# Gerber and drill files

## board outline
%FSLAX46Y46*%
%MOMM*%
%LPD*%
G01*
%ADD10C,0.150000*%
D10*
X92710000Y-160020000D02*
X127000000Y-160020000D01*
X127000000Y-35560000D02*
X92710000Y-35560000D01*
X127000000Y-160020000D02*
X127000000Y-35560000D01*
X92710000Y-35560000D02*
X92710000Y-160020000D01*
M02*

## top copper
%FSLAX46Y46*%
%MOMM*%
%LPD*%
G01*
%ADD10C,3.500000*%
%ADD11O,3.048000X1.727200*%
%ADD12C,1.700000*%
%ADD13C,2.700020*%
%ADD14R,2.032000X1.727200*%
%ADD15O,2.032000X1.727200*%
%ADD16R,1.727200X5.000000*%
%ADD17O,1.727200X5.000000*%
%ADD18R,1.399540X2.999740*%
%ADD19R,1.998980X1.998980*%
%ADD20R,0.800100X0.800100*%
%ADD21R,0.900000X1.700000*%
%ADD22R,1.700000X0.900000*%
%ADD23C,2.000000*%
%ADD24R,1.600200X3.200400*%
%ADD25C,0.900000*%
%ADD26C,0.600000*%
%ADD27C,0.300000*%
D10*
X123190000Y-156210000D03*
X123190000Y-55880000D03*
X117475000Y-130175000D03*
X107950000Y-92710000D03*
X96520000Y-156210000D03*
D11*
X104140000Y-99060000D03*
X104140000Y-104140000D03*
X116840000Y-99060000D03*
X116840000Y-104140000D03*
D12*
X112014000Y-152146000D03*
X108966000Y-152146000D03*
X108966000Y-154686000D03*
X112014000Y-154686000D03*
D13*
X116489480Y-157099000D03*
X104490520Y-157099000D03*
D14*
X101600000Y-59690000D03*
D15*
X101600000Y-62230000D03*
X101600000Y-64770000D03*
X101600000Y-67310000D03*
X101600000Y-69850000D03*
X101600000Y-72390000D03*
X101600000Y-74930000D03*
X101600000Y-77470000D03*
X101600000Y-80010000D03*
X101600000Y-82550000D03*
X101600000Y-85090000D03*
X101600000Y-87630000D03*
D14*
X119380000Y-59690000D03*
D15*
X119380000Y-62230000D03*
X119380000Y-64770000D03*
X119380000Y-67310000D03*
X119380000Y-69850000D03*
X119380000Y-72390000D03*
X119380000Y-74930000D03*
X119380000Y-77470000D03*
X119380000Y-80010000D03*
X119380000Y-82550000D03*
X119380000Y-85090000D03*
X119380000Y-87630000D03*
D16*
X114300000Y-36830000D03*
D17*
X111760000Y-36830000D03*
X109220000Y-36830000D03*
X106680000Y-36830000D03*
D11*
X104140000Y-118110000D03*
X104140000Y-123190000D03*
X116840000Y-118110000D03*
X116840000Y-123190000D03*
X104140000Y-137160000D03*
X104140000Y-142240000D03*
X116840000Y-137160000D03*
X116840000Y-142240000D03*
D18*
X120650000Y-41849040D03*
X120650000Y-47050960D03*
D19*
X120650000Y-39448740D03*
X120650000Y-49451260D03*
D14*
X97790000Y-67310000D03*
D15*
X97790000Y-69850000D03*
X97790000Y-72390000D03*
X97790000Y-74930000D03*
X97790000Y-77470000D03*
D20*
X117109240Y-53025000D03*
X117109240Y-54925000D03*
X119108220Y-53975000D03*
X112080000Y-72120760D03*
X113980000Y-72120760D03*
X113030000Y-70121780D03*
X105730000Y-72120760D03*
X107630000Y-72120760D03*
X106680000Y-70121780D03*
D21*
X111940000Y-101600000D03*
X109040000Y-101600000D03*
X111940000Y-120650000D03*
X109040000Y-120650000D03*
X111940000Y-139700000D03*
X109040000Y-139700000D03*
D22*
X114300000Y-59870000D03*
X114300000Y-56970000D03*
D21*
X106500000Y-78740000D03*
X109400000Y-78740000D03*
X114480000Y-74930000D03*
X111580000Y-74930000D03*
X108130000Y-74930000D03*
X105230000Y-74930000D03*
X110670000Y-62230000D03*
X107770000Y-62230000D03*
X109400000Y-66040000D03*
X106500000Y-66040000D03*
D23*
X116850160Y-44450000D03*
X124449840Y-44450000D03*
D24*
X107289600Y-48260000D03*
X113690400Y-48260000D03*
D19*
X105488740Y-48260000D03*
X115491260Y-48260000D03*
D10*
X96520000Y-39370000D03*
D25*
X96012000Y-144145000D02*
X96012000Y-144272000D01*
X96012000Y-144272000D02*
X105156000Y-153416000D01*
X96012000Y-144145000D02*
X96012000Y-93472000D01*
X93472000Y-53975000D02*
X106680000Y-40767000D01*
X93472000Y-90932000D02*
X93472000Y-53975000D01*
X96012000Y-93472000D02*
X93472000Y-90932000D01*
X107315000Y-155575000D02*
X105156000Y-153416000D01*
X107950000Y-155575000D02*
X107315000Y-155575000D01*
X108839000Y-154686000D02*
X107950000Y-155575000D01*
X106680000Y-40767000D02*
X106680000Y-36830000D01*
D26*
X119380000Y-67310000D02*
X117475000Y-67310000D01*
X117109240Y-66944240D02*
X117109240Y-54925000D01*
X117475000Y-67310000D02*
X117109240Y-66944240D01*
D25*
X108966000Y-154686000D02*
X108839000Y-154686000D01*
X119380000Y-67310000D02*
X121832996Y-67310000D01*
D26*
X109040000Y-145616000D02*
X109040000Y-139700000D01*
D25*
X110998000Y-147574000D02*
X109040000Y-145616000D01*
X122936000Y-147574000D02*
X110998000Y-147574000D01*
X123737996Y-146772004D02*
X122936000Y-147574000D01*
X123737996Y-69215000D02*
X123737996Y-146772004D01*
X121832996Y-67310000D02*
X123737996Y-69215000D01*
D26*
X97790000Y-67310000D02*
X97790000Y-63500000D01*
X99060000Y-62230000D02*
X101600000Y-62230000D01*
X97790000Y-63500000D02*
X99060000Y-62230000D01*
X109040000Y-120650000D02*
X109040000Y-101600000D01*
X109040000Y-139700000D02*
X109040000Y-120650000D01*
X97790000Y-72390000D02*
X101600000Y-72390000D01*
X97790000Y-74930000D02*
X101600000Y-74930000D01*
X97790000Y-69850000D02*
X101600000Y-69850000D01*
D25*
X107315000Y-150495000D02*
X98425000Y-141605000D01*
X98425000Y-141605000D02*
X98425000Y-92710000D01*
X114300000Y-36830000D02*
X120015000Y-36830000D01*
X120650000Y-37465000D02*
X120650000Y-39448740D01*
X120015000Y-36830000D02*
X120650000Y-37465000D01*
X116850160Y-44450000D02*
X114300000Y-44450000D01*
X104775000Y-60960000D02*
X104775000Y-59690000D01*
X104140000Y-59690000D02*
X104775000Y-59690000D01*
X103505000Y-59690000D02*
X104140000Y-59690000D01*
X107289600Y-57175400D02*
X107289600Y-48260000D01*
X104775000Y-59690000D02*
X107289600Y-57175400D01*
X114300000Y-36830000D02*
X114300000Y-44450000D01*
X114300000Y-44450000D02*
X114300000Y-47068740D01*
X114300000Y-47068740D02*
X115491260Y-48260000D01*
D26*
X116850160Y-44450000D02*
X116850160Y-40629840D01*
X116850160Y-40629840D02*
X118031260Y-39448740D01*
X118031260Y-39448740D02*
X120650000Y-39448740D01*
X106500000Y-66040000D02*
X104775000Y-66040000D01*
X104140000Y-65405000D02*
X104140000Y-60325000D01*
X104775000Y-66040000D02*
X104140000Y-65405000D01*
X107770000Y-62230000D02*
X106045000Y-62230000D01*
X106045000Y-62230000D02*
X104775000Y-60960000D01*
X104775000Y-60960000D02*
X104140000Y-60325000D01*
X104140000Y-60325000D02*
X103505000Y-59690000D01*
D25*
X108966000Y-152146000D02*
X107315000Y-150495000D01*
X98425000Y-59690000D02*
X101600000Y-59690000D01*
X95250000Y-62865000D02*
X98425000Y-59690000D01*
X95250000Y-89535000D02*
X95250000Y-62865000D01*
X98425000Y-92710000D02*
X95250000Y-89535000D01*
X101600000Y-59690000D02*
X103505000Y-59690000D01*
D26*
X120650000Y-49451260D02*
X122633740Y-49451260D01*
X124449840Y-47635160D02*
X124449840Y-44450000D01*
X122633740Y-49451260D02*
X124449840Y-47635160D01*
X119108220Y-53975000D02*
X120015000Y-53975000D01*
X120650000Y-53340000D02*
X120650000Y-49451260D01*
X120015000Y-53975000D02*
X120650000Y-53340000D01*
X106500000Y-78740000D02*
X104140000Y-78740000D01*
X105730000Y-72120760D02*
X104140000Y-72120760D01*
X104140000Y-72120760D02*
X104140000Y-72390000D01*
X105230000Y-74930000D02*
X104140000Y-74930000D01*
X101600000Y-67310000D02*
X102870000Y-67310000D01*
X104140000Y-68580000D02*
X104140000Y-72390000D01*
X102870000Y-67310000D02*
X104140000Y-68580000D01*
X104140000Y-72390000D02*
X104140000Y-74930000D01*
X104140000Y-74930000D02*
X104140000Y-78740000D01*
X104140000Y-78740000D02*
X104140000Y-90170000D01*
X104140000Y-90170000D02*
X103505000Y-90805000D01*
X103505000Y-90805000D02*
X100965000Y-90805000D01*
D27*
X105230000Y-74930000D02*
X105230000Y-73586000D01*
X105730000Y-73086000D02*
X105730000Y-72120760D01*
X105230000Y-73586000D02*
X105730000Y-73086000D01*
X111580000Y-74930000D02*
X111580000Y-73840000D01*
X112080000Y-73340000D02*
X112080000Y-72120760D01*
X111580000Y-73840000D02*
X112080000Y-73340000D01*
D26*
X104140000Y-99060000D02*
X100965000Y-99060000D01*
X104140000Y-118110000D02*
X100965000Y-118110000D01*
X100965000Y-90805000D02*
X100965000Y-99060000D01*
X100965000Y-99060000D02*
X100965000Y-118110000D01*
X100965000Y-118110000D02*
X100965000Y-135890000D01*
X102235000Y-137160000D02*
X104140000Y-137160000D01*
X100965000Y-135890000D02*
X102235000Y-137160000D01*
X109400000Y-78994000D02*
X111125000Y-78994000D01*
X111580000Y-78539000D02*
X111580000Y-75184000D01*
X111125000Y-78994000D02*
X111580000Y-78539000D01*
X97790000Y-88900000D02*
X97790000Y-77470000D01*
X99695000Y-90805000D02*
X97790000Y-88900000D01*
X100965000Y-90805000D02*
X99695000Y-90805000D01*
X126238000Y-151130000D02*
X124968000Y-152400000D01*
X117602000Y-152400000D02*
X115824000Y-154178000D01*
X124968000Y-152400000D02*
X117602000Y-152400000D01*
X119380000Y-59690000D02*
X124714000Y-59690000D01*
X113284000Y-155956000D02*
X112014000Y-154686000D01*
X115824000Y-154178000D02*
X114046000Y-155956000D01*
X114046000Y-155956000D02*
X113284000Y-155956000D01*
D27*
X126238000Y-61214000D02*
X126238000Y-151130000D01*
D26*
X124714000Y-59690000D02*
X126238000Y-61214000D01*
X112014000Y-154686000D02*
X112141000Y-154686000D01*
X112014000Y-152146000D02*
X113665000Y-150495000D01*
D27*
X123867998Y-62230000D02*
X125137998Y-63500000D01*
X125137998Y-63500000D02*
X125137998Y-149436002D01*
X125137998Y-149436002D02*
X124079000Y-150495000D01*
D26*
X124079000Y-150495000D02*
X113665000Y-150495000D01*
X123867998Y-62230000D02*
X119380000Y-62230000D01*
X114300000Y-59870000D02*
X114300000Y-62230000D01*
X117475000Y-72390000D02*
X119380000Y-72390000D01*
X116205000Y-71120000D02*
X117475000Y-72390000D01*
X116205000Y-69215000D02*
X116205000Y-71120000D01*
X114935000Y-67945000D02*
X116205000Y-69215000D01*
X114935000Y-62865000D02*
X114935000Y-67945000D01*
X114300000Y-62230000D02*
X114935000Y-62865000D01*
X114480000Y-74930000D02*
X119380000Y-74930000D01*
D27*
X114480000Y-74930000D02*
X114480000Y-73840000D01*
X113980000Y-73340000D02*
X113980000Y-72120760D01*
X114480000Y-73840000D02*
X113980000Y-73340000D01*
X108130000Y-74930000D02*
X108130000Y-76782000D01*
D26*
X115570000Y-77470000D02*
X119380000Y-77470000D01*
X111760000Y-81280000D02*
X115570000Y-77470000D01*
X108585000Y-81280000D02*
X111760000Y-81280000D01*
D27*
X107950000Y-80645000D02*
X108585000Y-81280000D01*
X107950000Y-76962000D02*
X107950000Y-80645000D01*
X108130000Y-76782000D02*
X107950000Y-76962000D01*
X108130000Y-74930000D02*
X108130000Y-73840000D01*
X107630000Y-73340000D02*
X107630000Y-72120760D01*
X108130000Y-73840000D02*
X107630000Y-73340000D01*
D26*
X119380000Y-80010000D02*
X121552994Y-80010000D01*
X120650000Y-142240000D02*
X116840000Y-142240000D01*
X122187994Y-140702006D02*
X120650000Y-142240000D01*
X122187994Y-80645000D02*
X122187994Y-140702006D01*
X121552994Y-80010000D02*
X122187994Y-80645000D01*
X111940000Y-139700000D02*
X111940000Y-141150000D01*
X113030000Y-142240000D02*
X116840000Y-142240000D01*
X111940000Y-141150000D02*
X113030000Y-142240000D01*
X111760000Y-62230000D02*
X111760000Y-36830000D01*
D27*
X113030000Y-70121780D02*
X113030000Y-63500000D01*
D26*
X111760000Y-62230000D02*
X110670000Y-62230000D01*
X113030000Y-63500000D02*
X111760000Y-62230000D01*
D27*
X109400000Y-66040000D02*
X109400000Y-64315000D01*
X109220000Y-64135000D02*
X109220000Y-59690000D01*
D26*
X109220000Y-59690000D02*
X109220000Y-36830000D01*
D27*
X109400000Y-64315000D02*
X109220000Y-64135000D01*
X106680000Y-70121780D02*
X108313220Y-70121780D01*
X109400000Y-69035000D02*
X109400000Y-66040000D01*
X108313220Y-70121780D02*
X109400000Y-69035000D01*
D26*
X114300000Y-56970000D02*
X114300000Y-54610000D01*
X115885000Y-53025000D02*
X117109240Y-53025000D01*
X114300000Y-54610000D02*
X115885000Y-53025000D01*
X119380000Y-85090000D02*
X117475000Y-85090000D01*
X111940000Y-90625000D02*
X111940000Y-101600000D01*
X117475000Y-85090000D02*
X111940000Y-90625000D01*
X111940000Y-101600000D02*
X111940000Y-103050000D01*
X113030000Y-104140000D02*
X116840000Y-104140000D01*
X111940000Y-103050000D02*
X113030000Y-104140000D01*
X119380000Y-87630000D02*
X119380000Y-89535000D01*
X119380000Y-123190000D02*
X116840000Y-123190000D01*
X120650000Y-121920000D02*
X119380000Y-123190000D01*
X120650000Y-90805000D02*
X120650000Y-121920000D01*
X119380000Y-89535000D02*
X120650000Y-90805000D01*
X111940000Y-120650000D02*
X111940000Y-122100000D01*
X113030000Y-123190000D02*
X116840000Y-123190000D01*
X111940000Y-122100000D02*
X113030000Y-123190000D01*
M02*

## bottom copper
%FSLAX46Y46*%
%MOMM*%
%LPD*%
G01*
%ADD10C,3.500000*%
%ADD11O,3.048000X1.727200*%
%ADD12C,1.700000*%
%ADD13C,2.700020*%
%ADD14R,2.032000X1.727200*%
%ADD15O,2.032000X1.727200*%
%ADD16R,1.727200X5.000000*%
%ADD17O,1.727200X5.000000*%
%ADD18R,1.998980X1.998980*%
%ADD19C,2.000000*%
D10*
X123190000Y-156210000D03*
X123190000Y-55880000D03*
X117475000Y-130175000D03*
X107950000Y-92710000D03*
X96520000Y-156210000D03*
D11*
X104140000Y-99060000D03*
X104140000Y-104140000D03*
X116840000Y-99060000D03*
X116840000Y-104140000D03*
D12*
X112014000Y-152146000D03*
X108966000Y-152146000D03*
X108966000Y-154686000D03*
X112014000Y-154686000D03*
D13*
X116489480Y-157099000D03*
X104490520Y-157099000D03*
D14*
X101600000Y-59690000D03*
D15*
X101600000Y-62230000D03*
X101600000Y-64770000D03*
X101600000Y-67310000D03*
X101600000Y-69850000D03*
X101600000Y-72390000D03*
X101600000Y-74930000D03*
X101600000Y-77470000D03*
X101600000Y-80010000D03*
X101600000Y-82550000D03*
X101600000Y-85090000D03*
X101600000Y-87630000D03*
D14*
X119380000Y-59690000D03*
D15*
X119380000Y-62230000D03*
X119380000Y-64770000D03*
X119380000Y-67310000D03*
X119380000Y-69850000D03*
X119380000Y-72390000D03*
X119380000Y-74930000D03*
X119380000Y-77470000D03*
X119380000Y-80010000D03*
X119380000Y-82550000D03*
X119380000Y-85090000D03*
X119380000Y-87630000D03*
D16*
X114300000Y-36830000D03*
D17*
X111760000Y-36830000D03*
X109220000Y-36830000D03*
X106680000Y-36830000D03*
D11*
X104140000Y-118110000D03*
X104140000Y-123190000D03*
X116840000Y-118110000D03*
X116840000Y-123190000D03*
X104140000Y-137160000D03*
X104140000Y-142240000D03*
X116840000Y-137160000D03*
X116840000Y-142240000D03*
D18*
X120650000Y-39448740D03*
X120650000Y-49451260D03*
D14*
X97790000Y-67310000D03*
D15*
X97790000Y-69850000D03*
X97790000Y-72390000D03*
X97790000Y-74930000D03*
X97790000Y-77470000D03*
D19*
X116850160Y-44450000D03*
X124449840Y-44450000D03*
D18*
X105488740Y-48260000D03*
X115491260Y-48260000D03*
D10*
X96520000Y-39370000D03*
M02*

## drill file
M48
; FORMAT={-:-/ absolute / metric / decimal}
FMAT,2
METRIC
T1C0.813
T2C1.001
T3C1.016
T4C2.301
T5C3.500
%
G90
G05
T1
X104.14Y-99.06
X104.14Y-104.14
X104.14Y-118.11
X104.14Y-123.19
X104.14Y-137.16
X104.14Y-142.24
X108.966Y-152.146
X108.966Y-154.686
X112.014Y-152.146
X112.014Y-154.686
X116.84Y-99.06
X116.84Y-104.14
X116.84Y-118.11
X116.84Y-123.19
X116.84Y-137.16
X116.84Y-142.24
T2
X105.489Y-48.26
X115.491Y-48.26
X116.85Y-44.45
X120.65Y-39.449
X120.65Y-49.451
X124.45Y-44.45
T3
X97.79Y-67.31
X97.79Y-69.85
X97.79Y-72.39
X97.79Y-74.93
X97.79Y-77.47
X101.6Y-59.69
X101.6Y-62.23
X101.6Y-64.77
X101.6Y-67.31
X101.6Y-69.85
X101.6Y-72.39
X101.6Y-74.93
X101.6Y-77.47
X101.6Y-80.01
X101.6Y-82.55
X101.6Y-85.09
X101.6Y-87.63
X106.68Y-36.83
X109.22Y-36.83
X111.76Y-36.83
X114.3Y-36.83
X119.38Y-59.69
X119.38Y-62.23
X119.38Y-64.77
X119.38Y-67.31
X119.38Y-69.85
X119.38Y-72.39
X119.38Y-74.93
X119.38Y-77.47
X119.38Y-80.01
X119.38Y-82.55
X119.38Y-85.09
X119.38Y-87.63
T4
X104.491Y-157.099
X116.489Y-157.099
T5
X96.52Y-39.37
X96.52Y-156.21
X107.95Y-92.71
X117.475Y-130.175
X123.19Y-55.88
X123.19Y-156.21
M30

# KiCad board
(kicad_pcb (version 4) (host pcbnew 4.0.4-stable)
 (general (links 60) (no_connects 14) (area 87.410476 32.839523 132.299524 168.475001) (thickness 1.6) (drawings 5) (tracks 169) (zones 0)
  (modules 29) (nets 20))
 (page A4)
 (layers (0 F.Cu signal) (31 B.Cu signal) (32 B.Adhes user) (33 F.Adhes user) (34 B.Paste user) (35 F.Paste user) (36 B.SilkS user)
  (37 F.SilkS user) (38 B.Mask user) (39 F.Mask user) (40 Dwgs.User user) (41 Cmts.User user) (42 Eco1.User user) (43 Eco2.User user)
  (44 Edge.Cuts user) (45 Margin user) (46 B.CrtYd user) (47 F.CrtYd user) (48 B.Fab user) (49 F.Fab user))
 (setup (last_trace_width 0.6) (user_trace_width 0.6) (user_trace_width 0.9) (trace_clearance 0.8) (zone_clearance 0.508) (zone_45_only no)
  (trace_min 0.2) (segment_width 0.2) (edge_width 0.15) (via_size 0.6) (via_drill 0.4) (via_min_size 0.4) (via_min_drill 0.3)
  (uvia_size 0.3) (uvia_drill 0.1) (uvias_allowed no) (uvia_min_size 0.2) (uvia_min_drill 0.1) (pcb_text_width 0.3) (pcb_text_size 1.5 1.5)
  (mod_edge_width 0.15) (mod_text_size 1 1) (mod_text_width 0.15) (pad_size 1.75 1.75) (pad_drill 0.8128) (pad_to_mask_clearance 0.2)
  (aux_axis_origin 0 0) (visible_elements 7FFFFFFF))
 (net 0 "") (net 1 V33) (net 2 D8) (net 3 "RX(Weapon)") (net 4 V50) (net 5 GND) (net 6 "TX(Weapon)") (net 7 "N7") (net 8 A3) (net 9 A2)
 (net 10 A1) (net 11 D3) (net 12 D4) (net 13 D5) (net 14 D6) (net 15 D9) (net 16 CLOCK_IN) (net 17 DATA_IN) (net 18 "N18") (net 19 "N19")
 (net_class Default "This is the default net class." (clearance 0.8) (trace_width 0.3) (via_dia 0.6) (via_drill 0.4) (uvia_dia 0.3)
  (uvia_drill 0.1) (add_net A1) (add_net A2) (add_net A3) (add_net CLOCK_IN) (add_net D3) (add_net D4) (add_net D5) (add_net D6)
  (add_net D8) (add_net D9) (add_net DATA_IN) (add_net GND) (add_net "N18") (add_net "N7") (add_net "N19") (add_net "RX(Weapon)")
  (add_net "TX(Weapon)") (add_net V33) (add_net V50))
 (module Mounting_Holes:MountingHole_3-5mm (layer F.Cu) (at 123.19 156.21)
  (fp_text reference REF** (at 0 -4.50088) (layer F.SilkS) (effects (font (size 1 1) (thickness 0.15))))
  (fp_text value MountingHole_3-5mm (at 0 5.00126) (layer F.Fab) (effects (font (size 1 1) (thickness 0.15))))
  (pad 1 thru_hole circle (at 0 0) (size 3.5 3.5) (drill 3.5) (layers)))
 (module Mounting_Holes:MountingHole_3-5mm (layer F.Cu) (at 123.19 55.88)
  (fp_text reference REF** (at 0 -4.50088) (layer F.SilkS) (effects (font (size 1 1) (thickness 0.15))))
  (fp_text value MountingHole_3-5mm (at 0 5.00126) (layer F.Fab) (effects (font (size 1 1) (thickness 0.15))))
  (pad 1 thru_hole circle (at 0 0) (size 3.5 3.5) (drill 3.5) (layers)))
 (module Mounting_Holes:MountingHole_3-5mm (layer F.Cu) (at 117.475 130.175)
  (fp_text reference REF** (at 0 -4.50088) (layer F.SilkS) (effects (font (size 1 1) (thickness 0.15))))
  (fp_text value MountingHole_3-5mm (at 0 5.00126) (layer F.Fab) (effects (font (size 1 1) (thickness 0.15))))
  (pad 1 thru_hole circle (at 0 0) (size 3.5 3.5) (drill 3.5) (layers)))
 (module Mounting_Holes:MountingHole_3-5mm (layer F.Cu) (at 107.95 92.71)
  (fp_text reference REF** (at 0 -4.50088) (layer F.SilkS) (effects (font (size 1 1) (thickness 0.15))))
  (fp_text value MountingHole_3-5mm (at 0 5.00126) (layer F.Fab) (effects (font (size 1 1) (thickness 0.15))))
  (pad 1 thru_hole circle (at 0 0) (size 3.5 3.5) (drill 3.5) (layers)))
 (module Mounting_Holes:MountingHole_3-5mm (layer F.Cu) (at 96.52 156.21)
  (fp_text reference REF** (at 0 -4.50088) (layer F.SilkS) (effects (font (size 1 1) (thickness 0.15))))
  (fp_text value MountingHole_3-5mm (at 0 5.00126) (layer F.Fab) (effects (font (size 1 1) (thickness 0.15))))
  (pad 1 thru_hole circle (at 0 0) (size 3.5 3.5) (drill 3.5) (layers)))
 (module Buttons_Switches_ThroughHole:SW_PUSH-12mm (layer B.Cu) (at 110.49 101.6 180)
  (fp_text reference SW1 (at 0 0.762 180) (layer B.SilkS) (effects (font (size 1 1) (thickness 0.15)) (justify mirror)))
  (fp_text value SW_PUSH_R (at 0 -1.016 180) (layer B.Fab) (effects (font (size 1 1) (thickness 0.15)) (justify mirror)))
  (pad 1 thru_hole oval (at 6.35 2.54 180) (size 3.048 1.7272) (drill 0.8128) (layers *.Cu *.Mask) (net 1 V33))
  (pad 2 thru_hole oval (at 6.35 -2.54 180) (size 3.048 1.7272) (drill 0.8128) (layers *.Cu *.Mask) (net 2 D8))
  (pad 1 thru_hole oval (at -6.35 2.54 180) (size 3.048 1.7272) (drill 0.8128) (layers *.Cu *.Mask) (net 1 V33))
  (pad 2 thru_hole oval (at -6.35 -2.54 180) (size 3.048 1.7272) (drill 0.8128) (layers *.Cu *.Mask) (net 2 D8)))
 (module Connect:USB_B (layer B.Cu) (at 109.22 152.4 270)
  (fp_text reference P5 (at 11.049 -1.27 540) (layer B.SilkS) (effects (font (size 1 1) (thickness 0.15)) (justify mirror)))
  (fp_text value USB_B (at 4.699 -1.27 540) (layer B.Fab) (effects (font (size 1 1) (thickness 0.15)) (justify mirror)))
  (pad 2 thru_hole circle (at -0.254 -2.794) (size 1.7 1.7) (drill 0.8128) (layers *.Cu *.Mask) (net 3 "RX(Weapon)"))
  (pad 1 thru_hole circle (at -0.254 0.254) (size 1.7 1.7) (drill 0.8128) (layers *.Cu *.Mask) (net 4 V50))
  (pad 4 thru_hole circle (at 2.286 0.254) (size 1.7 1.7) (drill 0.8128) (layers *.Cu *.Mask) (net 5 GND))
  (pad 3 thru_hole circle (at 2.286 -2.794) (size 1.7 1.7) (drill 0.8128) (layers *.Cu *.Mask) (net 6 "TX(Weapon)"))
  (pad 5 thru_hole circle (at 4.699 -7.26948) (size 2.70002 2.70002) (drill 2.30124) (layers *.Cu *.Mask) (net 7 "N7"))
  (pad 5 thru_hole circle (at 4.699 4.72948) (size 2.70002 2.70002) (drill 2.30124) (layers *.Cu *.Mask) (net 7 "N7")))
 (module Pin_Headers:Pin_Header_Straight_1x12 (layer B.Cu) (at 101.6 59.69 180)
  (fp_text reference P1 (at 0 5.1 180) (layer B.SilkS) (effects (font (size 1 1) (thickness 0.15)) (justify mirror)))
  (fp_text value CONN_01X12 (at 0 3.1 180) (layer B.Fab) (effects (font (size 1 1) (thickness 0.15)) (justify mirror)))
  (pad 1 thru_hole rect (at 0 0 180) (size 2.032 1.7272) (drill 1.016) (layers *.Cu *.Mask) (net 4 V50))
  (pad 2 thru_hole oval (at 0 -2.54 180) (size 2.032 1.7272) (drill 1.016) (layers *.Cu *.Mask) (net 5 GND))
  (pad 3 thru_hole oval (at 0 -5.08 180) (size 2.032 1.7272) (drill 1.016) (layers *.Cu *.Mask))
  (pad 4 thru_hole oval (at 0 -7.62 180) (size 2.032 1.7272) (drill 1.016) (layers *.Cu *.Mask) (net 1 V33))
  (pad 5 thru_hole oval (at 0 -10.16 180) (size 2.032 1.7272) (drill 1.016) (layers *.Cu *.Mask) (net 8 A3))
  (pad 6 thru_hole oval (at 0 -12.7 180) (size 2.032 1.7272) (drill 1.016) (layers *.Cu *.Mask) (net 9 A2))
  (pad 7 thru_hole oval (at 0 -15.24 180) (size 2.032 1.7272) (drill 1.016) (layers *.Cu *.Mask) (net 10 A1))
  (pad 8 thru_hole oval (at 0 -17.78 180) (size 2.032 1.7272) (drill 1.016) (layers *.Cu *.Mask))
  (pad 9 thru_hole oval (at 0 -20.32 180) (size 2.032 1.7272) (drill 1.016) (layers *.Cu *.Mask))
  (pad 10 thru_hole oval (at 0 -22.86 180) (size 2.032 1.7272) (drill 1.016) (layers *.Cu *.Mask))
  (pad 11 thru_hole oval (at 0 -25.4 180) (size 2.032 1.7272) (drill 1.016) (layers *.Cu *.Mask))
  (pad 12 thru_hole oval (at 0 -27.94 180) (size 2.032 1.7272) (drill 1.016) (layers *.Cu *.Mask)))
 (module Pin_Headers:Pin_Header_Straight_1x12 (layer B.Cu) (at 119.38 59.69 180)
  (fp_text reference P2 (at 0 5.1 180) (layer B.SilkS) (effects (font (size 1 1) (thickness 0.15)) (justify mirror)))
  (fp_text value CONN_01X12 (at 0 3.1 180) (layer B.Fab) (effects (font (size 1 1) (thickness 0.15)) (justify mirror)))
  (pad 1 thru_hole rect (at 0 0 180) (size 2.032 1.7272) (drill 1.016) (layers *.Cu *.Mask) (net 6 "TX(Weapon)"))
  (pad 2 thru_hole oval (at 0 -2.54 180) (size 2.032 1.7272) (drill 1.016) (layers *.Cu *.Mask) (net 3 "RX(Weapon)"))
  (pad 3 thru_hole oval (at 0 -5.08 180) (size 2.032 1.7272) (drill 1.016) (layers *.Cu *.Mask))
  (pad 4 thru_hole oval (at 0 -7.62 180) (size 2.032 1.7272) (drill 1.016) (layers *.Cu *.Mask) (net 5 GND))
  (pad 5 thru_hole oval (at 0 -10.16 180) (size 2.032 1.7272) (drill 1.016) (layers *.Cu *.Mask))
  (pad 6 thru_hole oval (at 0 -12.7 180) (size 2.032 1.7272) (drill 1.016) (layers *.Cu *.Mask) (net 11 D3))
  (pad 7 thru_hole oval (at 0 -15.24 180) (size 2.032 1.7272) (drill 1.016) (layers *.Cu *.Mask) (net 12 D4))
  (pad 8 thru_hole oval (at 0 -17.78 180) (size 2.032 1.7272) (drill 1.016) (layers *.Cu *.Mask) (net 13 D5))
  (pad 9 thru_hole oval (at 0 -20.32 180) (size 2.032 1.7272) (drill 1.016) (layers *.Cu *.Mask) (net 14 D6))
  (pad 10 thru_hole oval (at 0 -22.86 180) (size 2.032 1.7272) (drill 1.016) (layers *.Cu *.Mask))
  (pad 11 thru_hole oval (at 0 -25.4 180) (size 2.032 1.7272) (drill 1.016) (layers *.Cu *.Mask) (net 2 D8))
  (pad 12 thru_hole oval (at 0 -27.94 180) (size 2.032 1.7272) (drill 1.016) (layers *.Cu *.Mask) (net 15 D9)))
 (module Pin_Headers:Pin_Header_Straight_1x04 (layer F.Cu) (at 114.3 36.83 270)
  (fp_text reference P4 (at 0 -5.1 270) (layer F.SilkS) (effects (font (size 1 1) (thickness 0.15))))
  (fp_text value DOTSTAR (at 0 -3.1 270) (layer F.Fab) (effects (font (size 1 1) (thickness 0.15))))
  (pad 1 thru_hole rect (at 0 0 270) (size 5 1.7272) (drill 1.016) (layers *.Cu *.Mask) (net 4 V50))
  (pad 2 thru_hole oval (at 0 2.54 270) (size 5 1.7272) (drill 1.016) (layers *.Cu *.Mask) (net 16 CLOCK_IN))
  (pad 3 thru_hole oval (at 0 5.08 270) (size 5 1.7272) (drill 1.016) (layers *.Cu *.Mask) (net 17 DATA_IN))
  (pad 4 thru_hole oval (at 0 7.62 270) (size 5 1.7272) (drill 1.016) (layers *.Cu *.Mask) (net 5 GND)))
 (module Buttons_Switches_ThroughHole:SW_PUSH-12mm (layer B.Cu) (at 110.49 120.65 180)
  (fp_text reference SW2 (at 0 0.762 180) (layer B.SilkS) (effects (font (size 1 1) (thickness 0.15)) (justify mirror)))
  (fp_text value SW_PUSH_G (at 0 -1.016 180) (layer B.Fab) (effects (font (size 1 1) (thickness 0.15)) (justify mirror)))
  (pad 1 thru_hole oval (at 6.35 2.54 180) (size 3.048 1.7272) (drill 0.8128) (layers *.Cu *.Mask) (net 1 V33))
  (pad 2 thru_hole oval (at 6.35 -2.54 180) (size 3.048 1.7272) (drill 0.8128) (layers *.Cu *.Mask) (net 15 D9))
  (pad 1 thru_hole oval (at -6.35 2.54 180) (size 3.048 1.7272) (drill 0.8128) (layers *.Cu *.Mask) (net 1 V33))
  (pad 2 thru_hole oval (at -6.35 -2.54 180) (size 3.048 1.7272) (drill 0.8128) (layers *.Cu *.Mask) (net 15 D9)))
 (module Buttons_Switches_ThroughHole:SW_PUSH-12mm (layer B.Cu) (at 110.49 139.7 180)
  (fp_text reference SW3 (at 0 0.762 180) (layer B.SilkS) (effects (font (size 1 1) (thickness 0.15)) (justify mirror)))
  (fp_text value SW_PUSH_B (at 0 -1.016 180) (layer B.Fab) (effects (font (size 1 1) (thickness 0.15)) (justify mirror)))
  (pad 1 thru_hole oval (at 6.35 2.54 180) (size 3.048 1.7272) (drill 0.8128) (layers *.Cu *.Mask) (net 1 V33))
  (pad 2 thru_hole oval (at 6.35 -2.54 180) (size 3.048 1.7272) (drill 0.8128) (layers *.Cu *.Mask) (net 14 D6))
  (pad 1 thru_hole oval (at -6.35 2.54 180) (size 3.048 1.7272) (drill 0.8128) (layers *.Cu *.Mask) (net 1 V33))
  (pad 2 thru_hole oval (at -6.35 -2.54 180) (size 3.048 1.7272) (drill 0.8128) (layers *.Cu *.Mask) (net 14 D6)))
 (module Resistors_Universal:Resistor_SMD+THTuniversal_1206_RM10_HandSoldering (layer F.Cu) (at 120.65 44.45 270)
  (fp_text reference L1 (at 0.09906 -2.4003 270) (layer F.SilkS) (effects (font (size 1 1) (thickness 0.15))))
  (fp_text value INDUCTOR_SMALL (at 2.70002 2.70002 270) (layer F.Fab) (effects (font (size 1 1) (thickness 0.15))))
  (pad 1 smd rect (at -2.60096 0 270) (size 2.99974 1.39954) (layers F.Cu F.Paste F.Mask) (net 4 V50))
  (pad 2 smd rect (at 2.60096 0 270) (size 2.99974 1.39954) (layers F.Cu F.Paste F.Mask) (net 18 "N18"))
  (pad 1 thru_hole rect (at -5.00126 0 270) (size 1.99898 1.99898) (drill 1.00076) (layers *.Cu *.Mask F.SilkS) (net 4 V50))
  (pad 2 thru_hole rect (at 5.00126 0 270) (size 1.99898 1.99898) (drill 1.00076) (layers *.Cu *.Mask F.SilkS) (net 18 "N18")))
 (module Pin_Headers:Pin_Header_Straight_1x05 (layer B.Cu) (at 97.79 67.31 180)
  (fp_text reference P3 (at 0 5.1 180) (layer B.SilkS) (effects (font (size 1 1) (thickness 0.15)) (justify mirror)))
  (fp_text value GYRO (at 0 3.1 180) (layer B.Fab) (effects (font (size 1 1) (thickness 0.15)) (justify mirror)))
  (pad 1 thru_hole rect (at 0 0 180) (size 2.032 1.7272) (drill 1.016) (layers *.Cu *.Mask B.SilkS) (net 5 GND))
  (pad 2 thru_hole oval (at 0 -2.54 180) (size 2.032 1.7272) (drill 1.016) (layers *.Cu *.Mask B.SilkS) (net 8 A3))
  (pad 3 thru_hole oval (at 0 -5.08 180) (size 2.032 1.7272) (drill 1.016) (layers *.Cu *.Mask B.SilkS) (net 9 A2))
  (pad 4 thru_hole oval (at 0 -7.62 180) (size 2.032 1.7272) (drill 1.016) (layers *.Cu *.Mask B.SilkS) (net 10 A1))
  (pad 5 thru_hole oval (at 0 -10.16 180) (size 2.032 1.7272) (drill 1.016) (layers *.Cu *.Mask B.SilkS) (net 1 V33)))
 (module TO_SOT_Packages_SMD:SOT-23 (layer F.Cu) (at 118.11 53.975 270)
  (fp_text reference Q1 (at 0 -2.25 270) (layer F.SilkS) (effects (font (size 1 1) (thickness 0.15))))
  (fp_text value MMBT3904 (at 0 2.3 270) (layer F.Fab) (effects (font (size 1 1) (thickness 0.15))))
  (pad 1 smd rect (at -0.95 1.00076 270) (size 0.8001 0.8001) (layers F.Cu F.Paste F.Mask) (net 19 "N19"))
  (pad 2 smd rect (at 0.95 1.00076 270) (size 0.8001 0.8001) (layers F.Cu F.Paste F.Mask) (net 5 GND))
  (pad 3 smd rect (at 0 -0.99822 270) (size 0.8001 0.8001) (layers F.Cu F.Paste F.Mask) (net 18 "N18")))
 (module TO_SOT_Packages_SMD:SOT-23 (layer F.Cu) (at 113.03 71.12)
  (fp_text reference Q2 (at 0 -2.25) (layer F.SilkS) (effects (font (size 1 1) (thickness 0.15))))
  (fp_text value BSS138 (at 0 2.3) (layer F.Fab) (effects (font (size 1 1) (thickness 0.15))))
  (pad 1 smd rect (at -0.95 1.00076) (size 0.8001 0.8001) (layers F.Cu F.Paste F.Mask) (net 1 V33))
  (pad 2 smd rect (at 0.95 1.00076) (size 0.8001 0.8001) (layers F.Cu F.Paste F.Mask) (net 12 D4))
  (pad 3 smd rect (at 0 -0.99822) (size 0.8001 0.8001) (layers F.Cu F.Paste F.Mask) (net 16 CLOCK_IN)))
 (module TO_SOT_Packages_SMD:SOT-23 (layer F.Cu) (at 106.68 71.12)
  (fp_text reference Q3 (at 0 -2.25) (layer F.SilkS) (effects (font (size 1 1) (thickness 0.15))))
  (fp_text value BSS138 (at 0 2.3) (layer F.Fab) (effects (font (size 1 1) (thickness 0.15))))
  (pad 1 smd rect (at -0.95 1.00076) (size 0.8001 0.8001) (layers F.Cu F.Paste F.Mask) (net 1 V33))
  (pad 2 smd rect (at 0.95 1.00076) (size 0.8001 0.8001) (layers F.Cu F.Paste F.Mask) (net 13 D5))
  (pad 3 smd rect (at 0 -0.99822) (size 0.8001 0.8001) (layers F.Cu F.Paste F.Mask) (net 17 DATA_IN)))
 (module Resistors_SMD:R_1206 (layer F.Cu) (at 110.49 101.6 180)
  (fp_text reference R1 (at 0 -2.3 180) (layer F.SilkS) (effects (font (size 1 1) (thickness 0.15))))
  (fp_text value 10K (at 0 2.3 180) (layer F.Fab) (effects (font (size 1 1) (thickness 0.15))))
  (pad 1 smd rect (at -1.45 0 180) (size 0.9 1.7) (layers F.Cu F.Paste F.Mask) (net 2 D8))
  (pad 2 smd rect (at 1.45 0 180) (size 0.9 1.7) (layers F.Cu F.Paste F.Mask) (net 5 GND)))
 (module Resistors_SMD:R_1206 (layer F.Cu) (at 110.49 120.65 180)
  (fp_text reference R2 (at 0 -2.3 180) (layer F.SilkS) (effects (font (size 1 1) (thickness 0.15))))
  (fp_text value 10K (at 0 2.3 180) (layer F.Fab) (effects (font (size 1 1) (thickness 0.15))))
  (pad 1 smd rect (at -1.45 0 180) (size 0.9 1.7) (layers F.Cu F.Paste F.Mask) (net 15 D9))
  (pad 2 smd rect (at 1.45 0 180) (size 0.9 1.7) (layers F.Cu F.Paste F.Mask) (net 5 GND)))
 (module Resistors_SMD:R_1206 (layer F.Cu) (at 110.49 139.7 180)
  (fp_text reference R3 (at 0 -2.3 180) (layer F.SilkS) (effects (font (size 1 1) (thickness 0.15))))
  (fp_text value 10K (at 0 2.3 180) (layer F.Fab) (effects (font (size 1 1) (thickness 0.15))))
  (pad 1 smd rect (at -1.45 0 180) (size 0.9 1.7) (layers F.Cu F.Paste F.Mask) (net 14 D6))
  (pad 2 smd rect (at 1.45 0 180) (size 0.9 1.7) (layers F.Cu F.Paste F.Mask) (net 5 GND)))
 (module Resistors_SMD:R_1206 (layer F.Cu) (at 114.3 58.42 90)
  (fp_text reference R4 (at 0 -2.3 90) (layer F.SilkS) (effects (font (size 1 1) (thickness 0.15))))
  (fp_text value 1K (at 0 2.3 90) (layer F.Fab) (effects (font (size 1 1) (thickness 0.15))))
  (pad 1 smd rect (at -1.45 0 90) (size 0.9 1.7) (layers F.Cu F.Paste F.Mask) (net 11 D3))
  (pad 2 smd rect (at 1.45 0 90) (size 0.9 1.7) (layers F.Cu F.Paste F.Mask) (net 19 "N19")))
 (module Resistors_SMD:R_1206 (layer F.Cu) (at 107.95 78.74)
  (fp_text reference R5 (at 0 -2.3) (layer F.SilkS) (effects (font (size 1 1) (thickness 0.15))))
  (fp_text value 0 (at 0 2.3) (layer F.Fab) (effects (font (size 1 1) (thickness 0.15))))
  (pad 1 smd rect (at -1.45 0) (size 0.9 1.7) (layers F.Cu F.Paste F.Mask) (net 1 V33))
  (pad 2 smd rect (at 1.45 0) (size 0.9 1.7) (layers F.Cu F.Paste F.Mask) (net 1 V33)))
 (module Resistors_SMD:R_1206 (layer F.Cu) (at 113.03 74.93 180)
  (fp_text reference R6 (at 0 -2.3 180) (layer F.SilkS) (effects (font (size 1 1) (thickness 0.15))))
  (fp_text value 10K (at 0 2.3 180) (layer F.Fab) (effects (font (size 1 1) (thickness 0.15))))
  (pad 1 smd rect (at -1.45 0 180) (size 0.9 1.7) (layers F.Cu F.Paste F.Mask) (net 12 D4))
  (pad 2 smd rect (at 1.45 0 180) (size 0.9 1.7) (layers F.Cu F.Paste F.Mask) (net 1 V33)))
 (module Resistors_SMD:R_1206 (layer F.Cu) (at 106.68 74.93 180)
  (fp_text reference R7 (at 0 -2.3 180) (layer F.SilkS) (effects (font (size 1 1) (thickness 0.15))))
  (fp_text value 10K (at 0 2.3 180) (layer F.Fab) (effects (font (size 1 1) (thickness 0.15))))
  (pad 1 smd rect (at -1.45 0 180) (size 0.9 1.7) (layers F.Cu F.Paste F.Mask) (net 13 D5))
  (pad 2 smd rect (at 1.45 0 180) (size 0.9 1.7) (layers F.Cu F.Paste F.Mask) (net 1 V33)))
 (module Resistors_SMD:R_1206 (layer F.Cu) (at 109.22 62.23 180)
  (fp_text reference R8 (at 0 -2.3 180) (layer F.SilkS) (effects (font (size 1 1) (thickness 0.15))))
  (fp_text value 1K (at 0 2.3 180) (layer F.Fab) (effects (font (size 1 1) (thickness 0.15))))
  (pad 1 smd rect (at -1.45 0 180) (size 0.9 1.7) (layers F.Cu F.Paste F.Mask) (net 16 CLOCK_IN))
  (pad 2 smd rect (at 1.45 0 180) (size 0.9 1.7) (layers F.Cu F.Paste F.Mask) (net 4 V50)))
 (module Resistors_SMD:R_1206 (layer F.Cu) (at 107.95 66.04 180)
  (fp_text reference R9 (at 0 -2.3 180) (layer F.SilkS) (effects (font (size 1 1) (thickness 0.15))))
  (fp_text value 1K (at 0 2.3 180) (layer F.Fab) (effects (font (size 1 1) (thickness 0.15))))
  (pad 1 smd rect (at -1.45 0 180) (size 0.9 1.7) (layers F.Cu F.Paste F.Mask) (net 17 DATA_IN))
  (pad 2 smd rect (at 1.45 0 180) (size 0.9 1.7) (layers F.Cu F.Paste F.Mask) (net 4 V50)))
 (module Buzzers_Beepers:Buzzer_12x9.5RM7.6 (layer B.Cu) (at 120.65 44.45)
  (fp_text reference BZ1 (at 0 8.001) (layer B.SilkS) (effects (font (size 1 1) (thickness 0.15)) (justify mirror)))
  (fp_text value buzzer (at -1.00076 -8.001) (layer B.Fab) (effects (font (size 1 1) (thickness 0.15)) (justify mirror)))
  (pad 1 thru_hole circle (at -3.79984 0) (size 2 2) (drill 1.00076) (layers *.Cu *.Mask B.SilkS) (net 4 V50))
  (pad 2 thru_hole circle (at 3.79984 0) (size 2 2) (drill 1.00076) (layers *.Cu *.Mask B.SilkS) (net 18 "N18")))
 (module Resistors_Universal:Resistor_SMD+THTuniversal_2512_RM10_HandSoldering (layer F.Cu) (at 110.49 48.26)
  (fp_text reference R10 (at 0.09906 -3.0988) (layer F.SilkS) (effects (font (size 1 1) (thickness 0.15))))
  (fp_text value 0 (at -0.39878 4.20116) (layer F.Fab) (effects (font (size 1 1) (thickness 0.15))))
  (pad 1 smd rect (at -3.2004 0) (size 1.6002 3.2004) (layers F.Cu F.Paste F.Mask) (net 4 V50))
  (pad 2 smd rect (at 3.2004 0) (size 1.6002 3.2004) (layers F.Cu F.Paste F.Mask) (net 4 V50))
  (pad 1 thru_hole rect (at -5.00126 0 180) (size 1.99898 1.99898) (drill 1.00076) (layers *.Cu *.Mask F.SilkS) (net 4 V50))
  (pad 2 thru_hole rect (at 5.00126 0 180) (size 1.99898 1.99898) (drill 1.00076) (layers *.Cu *.Mask F.SilkS) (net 4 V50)))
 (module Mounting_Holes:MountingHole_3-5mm (layer F.Cu) (at 96.52 39.37)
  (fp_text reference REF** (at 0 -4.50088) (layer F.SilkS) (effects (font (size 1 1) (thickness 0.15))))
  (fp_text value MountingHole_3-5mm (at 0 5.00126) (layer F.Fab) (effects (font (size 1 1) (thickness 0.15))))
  (pad 1 thru_hole circle (at 0 0) (size 3.5 3.5) (drill 3.5) (layers)))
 (gr_line (start 92.71 160.02) (end 127 160.02) (angle 90) (layer Edge.Cuts) (width 0.15))
 (gr_line (start 127 35.56) (end 92.71 35.56) (angle 90) (layer Edge.Cuts) (width 0.15))
 (gr_line (start 127 160.02) (end 127 35.56) (angle 90) (layer Edge.Cuts) (width 0.15))
 (gr_line (start 92.71 35.56) (end 92.71 160.02) (angle 90) (layer Edge.Cuts) (width 0.15))
 (segment (start 96.012 144.145) (end 96.012 144.272) (width 0.9) (layer F.Cu) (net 5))
 (segment (start 96.012 144.272) (end 105.156 153.416) (width 0.9) (layer F.Cu) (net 5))
 (segment (start 96.012 144.145) (end 96.012 93.472) (width 0.9) (layer F.Cu) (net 5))
 (segment (start 93.472 53.975) (end 106.68 40.767) (width 0.9) (layer F.Cu) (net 5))
 (segment (start 93.472 90.932) (end 93.472 53.975) (width 0.9) (layer F.Cu) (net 5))
 (segment (start 96.012 93.472) (end 93.472 90.932) (width 0.9) (layer F.Cu) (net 5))
 (segment (start 107.315 155.575) (end 105.156 153.416) (width 0.9) (layer F.Cu) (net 5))
 (segment (start 107.95 155.575) (end 107.315 155.575) (width 0.9) (layer F.Cu) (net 5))
 (segment (start 108.839 154.686) (end 107.95 155.575) (width 0.9) (layer F.Cu) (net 5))
 (segment (start 106.68 40.767) (end 106.68 36.83) (width 0.9) (layer F.Cu) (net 5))
 (segment (start 119.38 67.31) (end 117.475 67.31) (width 0.6) (layer F.Cu) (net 5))
 (segment (start 117.10924 66.94424) (end 117.10924 54.925) (width 0.6) (layer F.Cu) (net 5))
 (segment (start 117.475 67.31) (end 117.10924 66.94424) (width 0.6) (layer F.Cu) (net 5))
 (segment (start 108.966 154.686) (end 108.839 154.686) (width 0.9) (layer F.Cu) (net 5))
 (segment (start 119.38 67.31) (end 121.832996 67.31) (width 0.9) (layer F.Cu) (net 5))
 (segment (start 109.04 145.616) (end 109.04 139.7) (width 0.6) (layer F.Cu) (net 5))
 (segment (start 110.998 147.574) (end 109.04 145.616) (width 0.9) (layer F.Cu) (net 5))
 (segment (start 122.936 147.574) (end 110.998 147.574) (width 0.9) (layer F.Cu) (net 5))
 (segment (start 123.737996 146.772004) (end 122.936 147.574) (width 0.9) (layer F.Cu) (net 5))
 (segment (start 123.737996 69.215) (end 123.737996 146.772004) (width 0.9) (layer F.Cu) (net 5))
 (segment (start 121.832996 67.31) (end 123.737996 69.215) (width 0.9) (layer F.Cu) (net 5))
 (segment (start 97.79 67.31) (end 97.79 63.5) (width 0.6) (layer F.Cu) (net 5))
 (segment (start 99.06 62.23) (end 101.6 62.23) (width 0.6) (layer F.Cu) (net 5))
 (segment (start 97.79 63.5) (end 99.06 62.23) (width 0.6) (layer F.Cu) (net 5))
 (segment (start 109.04 120.65) (end 109.04 101.6) (width 0.6) (layer F.Cu) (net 5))
 (segment (start 109.04 139.7) (end 109.04 120.65) (width 0.6) (layer F.Cu) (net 5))
 (segment (start 97.79 72.39) (end 101.6 72.39) (width 0.6) (layer F.Cu) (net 9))
 (segment (start 97.79 74.93) (end 101.6 74.93) (width 0.6) (layer F.Cu) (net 10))
 (segment (start 97.79 69.85) (end 101.6 69.85) (width 0.6) (layer F.Cu) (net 8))
 (segment (start 107.315 150.495) (end 98.425 141.605) (width 0.9) (layer F.Cu) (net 4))
 (segment (start 98.425 141.605) (end 98.425 92.71) (width 0.9) (layer F.Cu) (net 4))
 (segment (start 114.3 36.83) (end 120.015 36.83) (width 0.9) (layer F.Cu) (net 4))
 (segment (start 120.65 37.465) (end 120.65 39.44874) (width 0.9) (layer F.Cu) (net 4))
 (segment (start 120.015 36.83) (end 120.65 37.465) (width 0.9) (layer F.Cu) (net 4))
 (segment (start 116.85016 44.45) (end 114.3 44.45) (width 0.9) (layer F.Cu) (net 4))
 (segment (start 104.775 60.96) (end 104.775 59.69) (width 0.9) (layer F.Cu) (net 4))
 (segment (start 104.14 59.69) (end 104.775 59.69) (width 0.9) (layer F.Cu) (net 4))
 (segment (start 103.505 59.69) (end 104.14 59.69) (width 0.9) (layer F.Cu) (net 4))
 (segment (start 107.2896 57.1754) (end 107.2896 48.26) (width 0.9) (layer F.Cu) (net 4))
 (segment (start 104.775 59.69) (end 107.2896 57.1754) (width 0.9) (layer F.Cu) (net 4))
 (segment (start 114.3 36.83) (end 114.3 44.45) (width 0.9) (layer F.Cu) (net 4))
 (segment (start 114.3 44.45) (end 114.3 47.06874) (width 0.9) (layer F.Cu) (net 4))
 (segment (start 114.3 47.06874) (end 115.49126 48.26) (width 0.9) (layer F.Cu) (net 4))
 (segment (start 116.85016 44.45) (end 116.85016 40.62984) (width 0.6) (layer F.Cu) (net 4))
 (segment (start 116.85016 40.62984) (end 118.03126 39.44874) (width 0.6) (layer F.Cu) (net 4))
 (segment (start 118.03126 39.44874) (end 120.65 39.44874) (width 0.6) (layer F.Cu) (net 4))
 (segment (start 106.5 66.04) (end 104.775 66.04) (width 0.6) (layer F.Cu) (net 4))
 (segment (start 104.14 65.405) (end 104.14 60.325) (width 0.6) (layer F.Cu) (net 4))
 (segment (start 104.775 66.04) (end 104.14 65.405) (width 0.6) (layer F.Cu) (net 4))
 (segment (start 107.77 62.23) (end 106.045 62.23) (width 0.6) (layer F.Cu) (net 4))
 (segment (start 106.045 62.23) (end 104.775 60.96) (width 0.6) (layer F.Cu) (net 4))
 (segment (start 104.775 60.96) (end 104.14 60.325) (width 0.6) (layer F.Cu) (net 4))
 (segment (start 104.14 60.325) (end 103.505 59.69) (width 0.6) (layer F.Cu) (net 4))
 (segment (start 108.966 152.146) (end 107.315 150.495) (width 0.9) (layer F.Cu) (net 4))
 (segment (start 98.425 59.69) (end 101.6 59.69) (width 0.9) (layer F.Cu) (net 4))
 (segment (start 95.25 62.865) (end 98.425 59.69) (width 0.9) (layer F.Cu) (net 4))
 (segment (start 95.25 89.535) (end 95.25 62.865) (width 0.9) (layer F.Cu) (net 4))
 (segment (start 98.425 92.71) (end 95.25 89.535) (width 0.9) (layer F.Cu) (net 4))
 (segment (start 101.6 59.69) (end 103.505 59.69) (width 0.9) (layer F.Cu) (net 4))
 (segment (start 120.65 49.45126) (end 122.63374 49.45126) (width 0.6) (layer F.Cu) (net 18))
 (segment (start 124.44984 47.63516) (end 124.44984 44.45) (width 0.6) (layer F.Cu) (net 18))
 (segment (start 122.63374 49.45126) (end 124.44984 47.63516) (width 0.6) (layer F.Cu) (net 18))
 (segment (start 119.10822 53.975) (end 120.015 53.975) (width 0.6) (layer F.Cu) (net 18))
 (segment (start 120.65 53.34) (end 120.65 49.45126) (width 0.6) (layer F.Cu) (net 18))
 (segment (start 120.015 53.975) (end 120.65 53.34) (width 0.6) (layer F.Cu) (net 18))
 (segment (start 106.5 78.74) (end 104.14 78.74) (width 0.6) (layer F.Cu) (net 1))
 (segment (start 105.73 72.12076) (end 104.14 72.12076) (width 0.6) (layer F.Cu) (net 1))
 (segment (start 104.14 72.12076) (end 104.14 72.39) (width 0.6) (layer F.Cu) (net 1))
 (segment (start 105.23 74.93) (end 104.14 74.93) (width 0.6) (layer F.Cu) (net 1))
 (segment (start 101.6 67.31) (end 102.87 67.31) (width 0.6) (layer F.Cu) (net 1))
 (segment (start 104.14 68.58) (end 104.14 72.39) (width 0.6) (layer F.Cu) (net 1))
 (segment (start 102.87 67.31) (end 104.14 68.58) (width 0.6) (layer F.Cu) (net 1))
 (segment (start 104.14 72.39) (end 104.14 74.93) (width 0.6) (layer F.Cu) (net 1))
 (segment (start 104.14 74.93) (end 104.14 78.74) (width 0.6) (layer F.Cu) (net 1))
 (segment (start 104.14 78.74) (end 104.14 90.17) (width 0.6) (layer F.Cu) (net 1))
 (segment (start 104.14 90.17) (end 103.505 90.805) (width 0.6) (layer F.Cu) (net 1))
 (segment (start 103.505 90.805) (end 100.965 90.805) (width 0.6) (layer F.Cu) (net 1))
 (segment (start 105.23 74.93) (end 105.23 73.586) (width 0.3) (layer F.Cu) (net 1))
 (segment (start 105.73 73.086) (end 105.73 72.12076) (width 0.3) (layer F.Cu) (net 1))
 (segment (start 105.23 73.586) (end 105.73 73.086) (width 0.3) (layer F.Cu) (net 1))
 (segment (start 111.58 74.93) (end 111.58 73.84) (width 0.3) (layer F.Cu) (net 1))
 (segment (start 112.08 73.34) (end 112.08 72.12076) (width 0.3) (layer F.Cu) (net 1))
 (segment (start 111.58 73.84) (end 112.08 73.34) (width 0.3) (layer F.Cu) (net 1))
 (segment (start 104.14 99.06) (end 100.965 99.06) (width 0.6) (layer F.Cu) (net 1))
 (segment (start 104.14 118.11) (end 100.965 118.11) (width 0.6) (layer F.Cu) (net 1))
 (segment (start 100.965 90.805) (end 100.965 99.06) (width 0.6) (layer F.Cu) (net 1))
 (segment (start 100.965 99.06) (end 100.965 118.11) (width 0.6) (layer F.Cu) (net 1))
 (segment (start 100.965 118.11) (end 100.965 135.89) (width 0.6) (layer F.Cu) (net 1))
 (segment (start 102.235 137.16) (end 104.14 137.16) (width 0.6) (layer F.Cu) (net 1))
 (segment (start 100.965 135.89) (end 102.235 137.16) (width 0.6) (layer F.Cu) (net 1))
 (segment (start 109.4 78.994) (end 111.125 78.994) (width 0.6) (layer F.Cu) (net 1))
 (segment (start 111.58 78.539) (end 111.58 75.184) (width 0.6) (layer F.Cu) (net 1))
 (segment (start 111.125 78.994) (end 111.58 78.539) (width 0.6) (layer F.Cu) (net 1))
 (segment (start 97.79 88.9) (end 97.79 77.47) (width 0.6) (layer F.Cu) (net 1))
 (segment (start 99.695 90.805) (end 97.79 88.9) (width 0.6) (layer F.Cu) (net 1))
 (segment (start 100.965 90.805) (end 99.695 90.805) (width 0.6) (layer F.Cu) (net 1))
 (segment (start 126.238 151.13) (end 124.968 152.4) (width 0.6) (layer F.Cu) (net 6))
 (segment (start 117.602 152.4) (end 115.824 154.178) (width 0.6) (layer F.Cu) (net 6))
 (segment (start 124.968 152.4) (end 117.602 152.4) (width 0.6) (layer F.Cu) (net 6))
 (segment (start 119.38 59.69) (end 124.714 59.69) (width 0.6) (layer F.Cu) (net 6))
 (segment (start 113.284 155.956) (end 112.014 154.686) (width 0.6) (layer F.Cu) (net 6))
 (segment (start 115.824 154.178) (end 114.046 155.956) (width 0.6) (layer F.Cu) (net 6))
 (segment (start 114.046 155.956) (end 113.284 155.956) (width 0.6) (layer F.Cu) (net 6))
 (segment (start 126.238 61.214) (end 126.238 151.13) (width 0.3) (layer F.Cu) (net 6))
 (segment (start 124.714 59.69) (end 126.238 61.214) (width 0.6) (layer F.Cu) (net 6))
 (segment (start 112.014 154.686) (end 112.141 154.686) (width 0.6) (layer F.Cu) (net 6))
 (segment (start 112.014 152.146) (end 113.665 150.495) (width 0.6) (layer F.Cu) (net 3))
 (segment (start 123.867998 62.23) (end 125.137998 63.5) (width 0.3) (layer F.Cu) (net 3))
 (segment (start 125.137998 63.5) (end 125.137998 149.436002) (width 0.3) (layer F.Cu) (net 3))
 (segment (start 125.137998 149.436002) (end 124.079 150.495) (width 0.3) (layer F.Cu) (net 3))
 (segment (start 124.079 150.495) (end 113.665 150.495) (width 0.6) (layer F.Cu) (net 3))
 (segment (start 123.867998 62.23) (end 119.38 62.23) (width 0.6) (layer F.Cu) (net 3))
 (segment (start 114.3 59.87) (end 114.3 62.23) (width 0.6) (layer F.Cu) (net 11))
 (segment (start 117.475 72.39) (end 119.38 72.39) (width 0.6) (layer F.Cu) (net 11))
 (segment (start 116.205 71.12) (end 117.475 72.39) (width 0.6) (layer F.Cu) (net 11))
 (segment (start 116.205 69.215) (end 116.205 71.12) (width 0.6) (layer F.Cu) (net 11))
 (segment (start 114.935 67.945) (end 116.205 69.215) (width 0.6) (layer F.Cu) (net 11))
 (segment (start 114.935 62.865) (end 114.935 67.945) (width 0.6) (layer F.Cu) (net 11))
 (segment (start 114.3 62.23) (end 114.935 62.865) (width 0.6) (layer F.Cu) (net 11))
 (segment (start 114.48 74.93) (end 119.38 74.93) (width 0.6) (layer F.Cu) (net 12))
 (segment (start 114.48 74.93) (end 114.48 73.84) (width 0.3) (layer F.Cu) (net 12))
 (segment (start 113.98 73.34) (end 113.98 72.12076) (width 0.3) (layer F.Cu) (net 12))
 (segment (start 114.48 73.84) (end 113.98 73.34) (width 0.3) (layer F.Cu) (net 12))
 (segment (start 108.13 74.93) (end 108.13 76.782) (width 0.3) (layer F.Cu) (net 13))
 (segment (start 115.57 77.47) (end 119.38 77.47) (width 0.6) (layer F.Cu) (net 13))
 (segment (start 111.76 81.28) (end 115.57 77.47) (width 0.6) (layer F.Cu) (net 13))
 (segment (start 108.585 81.28) (end 111.76 81.28) (width 0.6) (layer F.Cu) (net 13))
 (segment (start 107.95 80.645) (end 108.585 81.28) (width 0.3) (layer F.Cu) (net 13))
 (segment (start 107.95 76.962) (end 107.95 80.645) (width 0.3) (layer F.Cu) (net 13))
 (segment (start 108.13 76.782) (end 107.95 76.962) (width 0.3) (layer F.Cu) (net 13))
 (segment (start 108.13 74.93) (end 108.13 73.84) (width 0.3) (layer F.Cu) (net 13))
 (segment (start 107.63 73.34) (end 107.63 72.12076) (width 0.3) (layer F.Cu) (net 13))
 (segment (start 108.13 73.84) (end 107.63 73.34) (width 0.3) (layer F.Cu) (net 13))
 (segment (start 119.38 80.01) (end 121.552994 80.01) (width 0.6) (layer F.Cu) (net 14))
 (segment (start 120.65 142.24) (end 116.84 142.24) (width 0.6) (layer F.Cu) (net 14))
 (segment (start 122.187994 140.702006) (end 120.65 142.24) (width 0.6) (layer F.Cu) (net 14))
 (segment (start 122.187994 80.645) (end 122.187994 140.702006) (width 0.6) (layer F.Cu) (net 14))
 (segment (start 121.552994 80.01) (end 122.187994 80.645) (width 0.6) (layer F.Cu) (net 14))
 (segment (start 111.94 139.7) (end 111.94 141.15) (width 0.6) (layer F.Cu) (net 14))
 (segment (start 113.03 142.24) (end 116.84 142.24) (width 0.6) (layer F.Cu) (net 14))
 (segment (start 111.94 141.15) (end 113.03 142.24) (width 0.6) (layer F.Cu) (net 14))
 (segment (start 111.76 62.23) (end 111.76 36.83) (width 0.6) (layer F.Cu) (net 16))
 (segment (start 113.03 70.12178) (end 113.03 63.5) (width 0.3) (layer F.Cu) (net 16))
 (segment (start 111.76 62.23) (end 110.67 62.23) (width 0.6) (layer F.Cu) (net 16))
 (segment (start 113.03 63.5) (end 111.76 62.23) (width 0.6) (layer F.Cu) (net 16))
 (segment (start 109.4 66.04) (end 109.4 64.315) (width 0.3) (layer F.Cu) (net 17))
 (segment (start 109.22 64.135) (end 109.22 59.69) (width 0.3) (layer F.Cu) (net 17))
 (segment (start 109.22 59.69) (end 109.22 36.83) (width 0.6) (layer F.Cu) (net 17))
 (segment (start 109.4 64.315) (end 109.22 64.135) (width 0.3) (layer F.Cu) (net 17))
 (segment (start 106.68 70.12178) (end 108.31322 70.12178) (width 0.3) (layer F.Cu) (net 17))
 (segment (start 109.4 69.035) (end 109.4 66.04) (width 0.3) (layer F.Cu) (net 17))
 (segment (start 108.31322 70.12178) (end 109.4 69.035) (width 0.3) (layer F.Cu) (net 17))
 (segment (start 114.3 56.97) (end 114.3 54.61) (width 0.6) (layer F.Cu) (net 19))
 (segment (start 115.885 53.025) (end 117.10924 53.025) (width 0.6) (layer F.Cu) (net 19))
 (segment (start 114.3 54.61) (end 115.885 53.025) (width 0.6) (layer F.Cu) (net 19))
 (segment (start 119.38 85.09) (end 117.475 85.09) (width 0.6) (layer F.Cu) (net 2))
 (segment (start 111.94 90.625) (end 111.94 101.6) (width 0.6) (layer F.Cu) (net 2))
 (segment (start 117.475 85.09) (end 111.94 90.625) (width 0.6) (layer F.Cu) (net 2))
 (segment (start 111.94 101.6) (end 111.94 103.05) (width 0.6) (layer F.Cu) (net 2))
 (segment (start 113.03 104.14) (end 116.84 104.14) (width 0.6) (layer F.Cu) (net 2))
 (segment (start 111.94 103.05) (end 113.03 104.14) (width 0.6) (layer F.Cu) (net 2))
 (segment (start 119.38 87.63) (end 119.38 89.535) (width 0.6) (layer F.Cu) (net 15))
 (segment (start 119.38 123.19) (end 116.84 123.19) (width 0.6) (layer F.Cu) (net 15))
 (segment (start 120.65 121.92) (end 119.38 123.19) (width 0.6) (layer F.Cu) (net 15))
 (segment (start 120.65 90.805) (end 120.65 121.92) (width 0.6) (layer F.Cu) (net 15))
 (segment (start 119.38 89.535) (end 120.65 90.805) (width 0.6) (layer F.Cu) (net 15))
 (segment (start 111.94 120.65) (end 111.94 122.1) (width 0.6) (layer F.Cu) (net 15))
 (segment (start 113.03 123.19) (end 116.84 123.19) (width 0.6) (layer F.Cu) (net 15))
 (segment (start 111.94 122.1) (end 113.03 123.19) (width 0.6) (layer F.Cu) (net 15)))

